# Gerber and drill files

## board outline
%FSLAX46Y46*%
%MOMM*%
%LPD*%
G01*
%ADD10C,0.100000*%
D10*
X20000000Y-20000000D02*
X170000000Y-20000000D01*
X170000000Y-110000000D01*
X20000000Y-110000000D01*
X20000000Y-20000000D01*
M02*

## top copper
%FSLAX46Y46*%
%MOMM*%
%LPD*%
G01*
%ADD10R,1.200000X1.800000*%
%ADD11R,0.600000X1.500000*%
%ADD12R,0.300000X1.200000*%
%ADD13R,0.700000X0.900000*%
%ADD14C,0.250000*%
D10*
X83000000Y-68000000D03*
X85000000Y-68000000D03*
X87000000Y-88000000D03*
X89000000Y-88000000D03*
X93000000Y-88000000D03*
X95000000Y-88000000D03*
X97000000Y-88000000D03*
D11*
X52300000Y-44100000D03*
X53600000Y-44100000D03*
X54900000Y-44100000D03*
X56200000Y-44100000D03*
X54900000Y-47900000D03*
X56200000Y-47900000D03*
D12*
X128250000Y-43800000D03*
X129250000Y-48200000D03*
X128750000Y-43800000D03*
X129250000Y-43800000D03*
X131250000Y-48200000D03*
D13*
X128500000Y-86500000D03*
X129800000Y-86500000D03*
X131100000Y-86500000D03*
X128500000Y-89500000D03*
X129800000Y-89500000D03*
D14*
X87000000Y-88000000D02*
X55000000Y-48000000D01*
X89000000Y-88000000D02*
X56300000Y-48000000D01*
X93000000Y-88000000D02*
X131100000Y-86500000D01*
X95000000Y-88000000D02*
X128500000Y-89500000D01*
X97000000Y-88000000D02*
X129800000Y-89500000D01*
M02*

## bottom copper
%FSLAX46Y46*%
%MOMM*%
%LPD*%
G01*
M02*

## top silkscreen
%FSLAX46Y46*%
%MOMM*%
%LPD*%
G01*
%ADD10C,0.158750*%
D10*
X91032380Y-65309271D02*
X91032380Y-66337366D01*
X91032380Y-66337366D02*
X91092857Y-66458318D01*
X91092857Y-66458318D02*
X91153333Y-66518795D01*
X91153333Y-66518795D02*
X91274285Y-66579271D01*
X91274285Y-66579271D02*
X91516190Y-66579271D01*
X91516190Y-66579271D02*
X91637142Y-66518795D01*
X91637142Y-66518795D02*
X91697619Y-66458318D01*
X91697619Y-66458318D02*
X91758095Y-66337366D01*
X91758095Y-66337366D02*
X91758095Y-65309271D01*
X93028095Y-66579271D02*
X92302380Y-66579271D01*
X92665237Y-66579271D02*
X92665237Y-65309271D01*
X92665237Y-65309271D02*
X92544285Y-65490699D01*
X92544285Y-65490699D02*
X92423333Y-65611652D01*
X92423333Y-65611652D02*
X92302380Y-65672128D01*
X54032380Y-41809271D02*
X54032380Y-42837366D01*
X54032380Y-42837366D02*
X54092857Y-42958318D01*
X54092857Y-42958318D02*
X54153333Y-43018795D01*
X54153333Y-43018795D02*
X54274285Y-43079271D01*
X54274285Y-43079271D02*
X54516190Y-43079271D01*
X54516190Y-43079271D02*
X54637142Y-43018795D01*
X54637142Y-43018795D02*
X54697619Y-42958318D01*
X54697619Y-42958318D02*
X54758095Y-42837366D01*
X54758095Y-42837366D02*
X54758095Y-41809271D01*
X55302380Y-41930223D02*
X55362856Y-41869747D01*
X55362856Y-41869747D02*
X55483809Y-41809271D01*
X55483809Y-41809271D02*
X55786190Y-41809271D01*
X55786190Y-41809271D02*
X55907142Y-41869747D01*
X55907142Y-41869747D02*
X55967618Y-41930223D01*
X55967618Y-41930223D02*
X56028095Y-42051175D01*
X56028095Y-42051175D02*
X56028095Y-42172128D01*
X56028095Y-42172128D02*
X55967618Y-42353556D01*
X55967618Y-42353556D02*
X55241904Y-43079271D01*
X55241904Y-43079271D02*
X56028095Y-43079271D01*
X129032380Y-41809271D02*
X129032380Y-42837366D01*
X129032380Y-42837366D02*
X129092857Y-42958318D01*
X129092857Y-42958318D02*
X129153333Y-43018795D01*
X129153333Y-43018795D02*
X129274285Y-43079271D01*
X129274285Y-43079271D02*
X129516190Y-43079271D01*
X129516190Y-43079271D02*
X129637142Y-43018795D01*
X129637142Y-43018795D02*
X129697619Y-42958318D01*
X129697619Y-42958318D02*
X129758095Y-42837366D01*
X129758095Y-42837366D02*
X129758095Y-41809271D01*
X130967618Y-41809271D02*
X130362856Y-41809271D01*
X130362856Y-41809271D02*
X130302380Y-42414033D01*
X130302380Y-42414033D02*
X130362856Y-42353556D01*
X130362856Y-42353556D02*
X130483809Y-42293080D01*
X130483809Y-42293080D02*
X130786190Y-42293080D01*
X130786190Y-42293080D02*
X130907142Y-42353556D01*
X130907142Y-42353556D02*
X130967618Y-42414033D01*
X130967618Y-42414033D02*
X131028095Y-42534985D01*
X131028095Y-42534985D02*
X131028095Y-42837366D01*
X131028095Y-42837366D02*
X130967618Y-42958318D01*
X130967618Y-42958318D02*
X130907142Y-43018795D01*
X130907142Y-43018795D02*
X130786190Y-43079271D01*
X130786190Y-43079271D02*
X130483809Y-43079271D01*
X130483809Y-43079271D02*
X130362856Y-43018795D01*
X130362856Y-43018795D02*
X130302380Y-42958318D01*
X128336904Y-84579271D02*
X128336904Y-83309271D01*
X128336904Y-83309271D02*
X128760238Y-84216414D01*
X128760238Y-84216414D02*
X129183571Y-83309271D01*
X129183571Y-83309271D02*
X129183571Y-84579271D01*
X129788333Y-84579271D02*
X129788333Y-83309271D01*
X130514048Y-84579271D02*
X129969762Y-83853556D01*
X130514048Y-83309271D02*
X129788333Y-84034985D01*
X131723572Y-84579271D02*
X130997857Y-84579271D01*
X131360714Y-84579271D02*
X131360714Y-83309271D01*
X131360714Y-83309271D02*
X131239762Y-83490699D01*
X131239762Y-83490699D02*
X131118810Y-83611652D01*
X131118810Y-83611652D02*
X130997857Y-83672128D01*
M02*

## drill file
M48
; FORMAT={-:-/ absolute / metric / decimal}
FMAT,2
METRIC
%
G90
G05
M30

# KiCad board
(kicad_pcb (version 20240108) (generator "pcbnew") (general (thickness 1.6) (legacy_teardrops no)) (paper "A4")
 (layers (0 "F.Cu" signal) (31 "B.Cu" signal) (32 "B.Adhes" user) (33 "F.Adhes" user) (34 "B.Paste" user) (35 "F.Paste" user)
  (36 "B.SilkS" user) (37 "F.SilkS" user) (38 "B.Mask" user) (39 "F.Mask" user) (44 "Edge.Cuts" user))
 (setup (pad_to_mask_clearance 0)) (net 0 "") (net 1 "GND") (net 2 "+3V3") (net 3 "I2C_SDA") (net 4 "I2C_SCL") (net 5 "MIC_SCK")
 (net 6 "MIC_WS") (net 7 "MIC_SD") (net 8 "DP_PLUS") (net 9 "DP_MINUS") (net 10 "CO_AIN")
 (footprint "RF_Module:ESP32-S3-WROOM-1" (layer "F.Cu") (at 92 78) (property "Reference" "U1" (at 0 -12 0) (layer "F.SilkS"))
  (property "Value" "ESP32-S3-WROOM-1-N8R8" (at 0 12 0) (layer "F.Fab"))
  (pad "1" smd rect (at -9 -10) (size 1.2 1.8) (layers "F.Cu" "F.Paste" "F.Mask") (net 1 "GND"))
  (pad "2" smd rect (at -7 -10) (size 1.2 1.8) (layers "F.Cu" "F.Paste" "F.Mask") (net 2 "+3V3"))
  (pad "15" smd rect (at -5 10) (size 1.2 1.8) (layers "F.Cu" "F.Paste" "F.Mask") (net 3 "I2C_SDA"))
  (pad "16" smd rect (at -3 10) (size 1.2 1.8) (layers "F.Cu" "F.Paste" "F.Mask") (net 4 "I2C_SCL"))
  (pad "12" smd rect (at 1 10) (size 1.2 1.8) (layers "F.Cu" "F.Paste" "F.Mask") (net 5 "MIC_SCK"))
  (pad "13" smd rect (at 3 10) (size 1.2 1.8) (layers "F.Cu" "F.Paste" "F.Mask") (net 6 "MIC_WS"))
  (pad "14" smd rect (at 5 10) (size 1.2 1.8) (layers "F.Cu" "F.Paste" "F.Mask") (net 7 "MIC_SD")))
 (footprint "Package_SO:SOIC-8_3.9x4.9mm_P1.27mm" (layer "F.Cu") (at 55 46) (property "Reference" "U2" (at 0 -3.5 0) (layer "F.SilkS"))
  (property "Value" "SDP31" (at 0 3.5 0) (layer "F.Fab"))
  (pad "1" smd rect (at -2.7 -1.9) (size 0.6 1.5) (layers "F.Cu" "F.Paste" "F.Mask") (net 2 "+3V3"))
  (pad "2" smd rect (at -1.4 -1.9) (size 0.6 1.5) (layers "F.Cu" "F.Paste" "F.Mask") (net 1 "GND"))
  (pad "3" smd rect (at -0.1 -1.9) (size 0.6 1.5) (layers "F.Cu" "F.Paste" "F.Mask") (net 3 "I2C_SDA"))
  (pad "4" smd rect (at 1.2 -1.9) (size 0.6 1.5) (layers "F.Cu" "F.Paste" "F.Mask") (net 4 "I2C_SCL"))
  (pad "5" smd rect (at -0.1 1.9) (size 0.6 1.5) (layers "F.Cu" "F.Paste" "F.Mask") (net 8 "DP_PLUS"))
  (pad "6" smd rect (at 1.2 1.9) (size 0.6 1.5) (layers "F.Cu" "F.Paste" "F.Mask") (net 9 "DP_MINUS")))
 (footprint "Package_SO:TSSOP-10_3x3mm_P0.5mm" (layer "F.Cu") (at 130 46) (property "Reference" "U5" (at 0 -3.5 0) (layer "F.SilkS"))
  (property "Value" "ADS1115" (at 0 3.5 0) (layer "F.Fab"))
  (pad "10" smd rect (at -1.75 -2.2) (size 0.3 1.2) (layers "F.Cu" "F.Paste" "F.Mask") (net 2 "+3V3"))
  (pad "3" smd rect (at -0.75 2.2) (size 0.3 1.2) (layers "F.Cu" "F.Paste" "F.Mask") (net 1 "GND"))
  (pad "9" smd rect (at -1.25 -2.2) (size 0.3 1.2) (layers "F.Cu" "F.Paste" "F.Mask") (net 3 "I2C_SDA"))
  (pad "8" smd rect (at -0.75 -2.2) (size 0.3 1.2) (layers "F.Cu" "F.Paste" "F.Mask") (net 4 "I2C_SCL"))
  (pad "4" smd rect (at 1.25 2.2) (size 0.3 1.2) (layers "F.Cu" "F.Paste" "F.Mask") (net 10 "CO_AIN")))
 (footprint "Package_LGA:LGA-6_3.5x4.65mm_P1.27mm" (layer "F.Cu") (at 130 88) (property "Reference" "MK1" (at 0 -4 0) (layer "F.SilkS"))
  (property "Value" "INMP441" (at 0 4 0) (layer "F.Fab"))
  (pad "1" smd rect (at -1.5 -1.5) (size 0.7 0.9) (layers "F.Cu" "F.Paste" "F.Mask") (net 2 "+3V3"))
  (pad "2" smd rect (at -0.2 -1.5) (size 0.7 0.9) (layers "F.Cu" "F.Paste" "F.Mask") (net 1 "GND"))
  (pad "3" smd rect (at 1.1 -1.5) (size 0.7 0.9) (layers "F.Cu" "F.Paste" "F.Mask") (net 5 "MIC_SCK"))
  (pad "4" smd rect (at -1.5 1.5) (size 0.7 0.9) (layers "F.Cu" "F.Paste" "F.Mask") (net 6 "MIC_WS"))
  (pad "5" smd rect (at -0.2 1.5) (size 0.7 0.9) (layers "F.Cu" "F.Paste" "F.Mask") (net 7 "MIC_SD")))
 (gr_rect (start 20 20) (end 170 110) (stroke (width 0.1) (type default)) (fill none) (layer "Edge.Cuts"))
 (segment (start 87 88) (end 55 48) (width 0.25) (layer "F.Cu") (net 3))
 (segment (start 89 88) (end 56.3 48) (width 0.25) (layer "F.Cu") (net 4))
 (segment (start 93 88) (end 131.1 86.5) (width 0.25) (layer "F.Cu") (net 5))
 (segment (start 95 88) (end 128.5 89.5) (width 0.25) (layer "F.Cu") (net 6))
 (segment (start 97 88) (end 129.8 89.5) (width 0.25) (layer "F.Cu") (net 7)))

